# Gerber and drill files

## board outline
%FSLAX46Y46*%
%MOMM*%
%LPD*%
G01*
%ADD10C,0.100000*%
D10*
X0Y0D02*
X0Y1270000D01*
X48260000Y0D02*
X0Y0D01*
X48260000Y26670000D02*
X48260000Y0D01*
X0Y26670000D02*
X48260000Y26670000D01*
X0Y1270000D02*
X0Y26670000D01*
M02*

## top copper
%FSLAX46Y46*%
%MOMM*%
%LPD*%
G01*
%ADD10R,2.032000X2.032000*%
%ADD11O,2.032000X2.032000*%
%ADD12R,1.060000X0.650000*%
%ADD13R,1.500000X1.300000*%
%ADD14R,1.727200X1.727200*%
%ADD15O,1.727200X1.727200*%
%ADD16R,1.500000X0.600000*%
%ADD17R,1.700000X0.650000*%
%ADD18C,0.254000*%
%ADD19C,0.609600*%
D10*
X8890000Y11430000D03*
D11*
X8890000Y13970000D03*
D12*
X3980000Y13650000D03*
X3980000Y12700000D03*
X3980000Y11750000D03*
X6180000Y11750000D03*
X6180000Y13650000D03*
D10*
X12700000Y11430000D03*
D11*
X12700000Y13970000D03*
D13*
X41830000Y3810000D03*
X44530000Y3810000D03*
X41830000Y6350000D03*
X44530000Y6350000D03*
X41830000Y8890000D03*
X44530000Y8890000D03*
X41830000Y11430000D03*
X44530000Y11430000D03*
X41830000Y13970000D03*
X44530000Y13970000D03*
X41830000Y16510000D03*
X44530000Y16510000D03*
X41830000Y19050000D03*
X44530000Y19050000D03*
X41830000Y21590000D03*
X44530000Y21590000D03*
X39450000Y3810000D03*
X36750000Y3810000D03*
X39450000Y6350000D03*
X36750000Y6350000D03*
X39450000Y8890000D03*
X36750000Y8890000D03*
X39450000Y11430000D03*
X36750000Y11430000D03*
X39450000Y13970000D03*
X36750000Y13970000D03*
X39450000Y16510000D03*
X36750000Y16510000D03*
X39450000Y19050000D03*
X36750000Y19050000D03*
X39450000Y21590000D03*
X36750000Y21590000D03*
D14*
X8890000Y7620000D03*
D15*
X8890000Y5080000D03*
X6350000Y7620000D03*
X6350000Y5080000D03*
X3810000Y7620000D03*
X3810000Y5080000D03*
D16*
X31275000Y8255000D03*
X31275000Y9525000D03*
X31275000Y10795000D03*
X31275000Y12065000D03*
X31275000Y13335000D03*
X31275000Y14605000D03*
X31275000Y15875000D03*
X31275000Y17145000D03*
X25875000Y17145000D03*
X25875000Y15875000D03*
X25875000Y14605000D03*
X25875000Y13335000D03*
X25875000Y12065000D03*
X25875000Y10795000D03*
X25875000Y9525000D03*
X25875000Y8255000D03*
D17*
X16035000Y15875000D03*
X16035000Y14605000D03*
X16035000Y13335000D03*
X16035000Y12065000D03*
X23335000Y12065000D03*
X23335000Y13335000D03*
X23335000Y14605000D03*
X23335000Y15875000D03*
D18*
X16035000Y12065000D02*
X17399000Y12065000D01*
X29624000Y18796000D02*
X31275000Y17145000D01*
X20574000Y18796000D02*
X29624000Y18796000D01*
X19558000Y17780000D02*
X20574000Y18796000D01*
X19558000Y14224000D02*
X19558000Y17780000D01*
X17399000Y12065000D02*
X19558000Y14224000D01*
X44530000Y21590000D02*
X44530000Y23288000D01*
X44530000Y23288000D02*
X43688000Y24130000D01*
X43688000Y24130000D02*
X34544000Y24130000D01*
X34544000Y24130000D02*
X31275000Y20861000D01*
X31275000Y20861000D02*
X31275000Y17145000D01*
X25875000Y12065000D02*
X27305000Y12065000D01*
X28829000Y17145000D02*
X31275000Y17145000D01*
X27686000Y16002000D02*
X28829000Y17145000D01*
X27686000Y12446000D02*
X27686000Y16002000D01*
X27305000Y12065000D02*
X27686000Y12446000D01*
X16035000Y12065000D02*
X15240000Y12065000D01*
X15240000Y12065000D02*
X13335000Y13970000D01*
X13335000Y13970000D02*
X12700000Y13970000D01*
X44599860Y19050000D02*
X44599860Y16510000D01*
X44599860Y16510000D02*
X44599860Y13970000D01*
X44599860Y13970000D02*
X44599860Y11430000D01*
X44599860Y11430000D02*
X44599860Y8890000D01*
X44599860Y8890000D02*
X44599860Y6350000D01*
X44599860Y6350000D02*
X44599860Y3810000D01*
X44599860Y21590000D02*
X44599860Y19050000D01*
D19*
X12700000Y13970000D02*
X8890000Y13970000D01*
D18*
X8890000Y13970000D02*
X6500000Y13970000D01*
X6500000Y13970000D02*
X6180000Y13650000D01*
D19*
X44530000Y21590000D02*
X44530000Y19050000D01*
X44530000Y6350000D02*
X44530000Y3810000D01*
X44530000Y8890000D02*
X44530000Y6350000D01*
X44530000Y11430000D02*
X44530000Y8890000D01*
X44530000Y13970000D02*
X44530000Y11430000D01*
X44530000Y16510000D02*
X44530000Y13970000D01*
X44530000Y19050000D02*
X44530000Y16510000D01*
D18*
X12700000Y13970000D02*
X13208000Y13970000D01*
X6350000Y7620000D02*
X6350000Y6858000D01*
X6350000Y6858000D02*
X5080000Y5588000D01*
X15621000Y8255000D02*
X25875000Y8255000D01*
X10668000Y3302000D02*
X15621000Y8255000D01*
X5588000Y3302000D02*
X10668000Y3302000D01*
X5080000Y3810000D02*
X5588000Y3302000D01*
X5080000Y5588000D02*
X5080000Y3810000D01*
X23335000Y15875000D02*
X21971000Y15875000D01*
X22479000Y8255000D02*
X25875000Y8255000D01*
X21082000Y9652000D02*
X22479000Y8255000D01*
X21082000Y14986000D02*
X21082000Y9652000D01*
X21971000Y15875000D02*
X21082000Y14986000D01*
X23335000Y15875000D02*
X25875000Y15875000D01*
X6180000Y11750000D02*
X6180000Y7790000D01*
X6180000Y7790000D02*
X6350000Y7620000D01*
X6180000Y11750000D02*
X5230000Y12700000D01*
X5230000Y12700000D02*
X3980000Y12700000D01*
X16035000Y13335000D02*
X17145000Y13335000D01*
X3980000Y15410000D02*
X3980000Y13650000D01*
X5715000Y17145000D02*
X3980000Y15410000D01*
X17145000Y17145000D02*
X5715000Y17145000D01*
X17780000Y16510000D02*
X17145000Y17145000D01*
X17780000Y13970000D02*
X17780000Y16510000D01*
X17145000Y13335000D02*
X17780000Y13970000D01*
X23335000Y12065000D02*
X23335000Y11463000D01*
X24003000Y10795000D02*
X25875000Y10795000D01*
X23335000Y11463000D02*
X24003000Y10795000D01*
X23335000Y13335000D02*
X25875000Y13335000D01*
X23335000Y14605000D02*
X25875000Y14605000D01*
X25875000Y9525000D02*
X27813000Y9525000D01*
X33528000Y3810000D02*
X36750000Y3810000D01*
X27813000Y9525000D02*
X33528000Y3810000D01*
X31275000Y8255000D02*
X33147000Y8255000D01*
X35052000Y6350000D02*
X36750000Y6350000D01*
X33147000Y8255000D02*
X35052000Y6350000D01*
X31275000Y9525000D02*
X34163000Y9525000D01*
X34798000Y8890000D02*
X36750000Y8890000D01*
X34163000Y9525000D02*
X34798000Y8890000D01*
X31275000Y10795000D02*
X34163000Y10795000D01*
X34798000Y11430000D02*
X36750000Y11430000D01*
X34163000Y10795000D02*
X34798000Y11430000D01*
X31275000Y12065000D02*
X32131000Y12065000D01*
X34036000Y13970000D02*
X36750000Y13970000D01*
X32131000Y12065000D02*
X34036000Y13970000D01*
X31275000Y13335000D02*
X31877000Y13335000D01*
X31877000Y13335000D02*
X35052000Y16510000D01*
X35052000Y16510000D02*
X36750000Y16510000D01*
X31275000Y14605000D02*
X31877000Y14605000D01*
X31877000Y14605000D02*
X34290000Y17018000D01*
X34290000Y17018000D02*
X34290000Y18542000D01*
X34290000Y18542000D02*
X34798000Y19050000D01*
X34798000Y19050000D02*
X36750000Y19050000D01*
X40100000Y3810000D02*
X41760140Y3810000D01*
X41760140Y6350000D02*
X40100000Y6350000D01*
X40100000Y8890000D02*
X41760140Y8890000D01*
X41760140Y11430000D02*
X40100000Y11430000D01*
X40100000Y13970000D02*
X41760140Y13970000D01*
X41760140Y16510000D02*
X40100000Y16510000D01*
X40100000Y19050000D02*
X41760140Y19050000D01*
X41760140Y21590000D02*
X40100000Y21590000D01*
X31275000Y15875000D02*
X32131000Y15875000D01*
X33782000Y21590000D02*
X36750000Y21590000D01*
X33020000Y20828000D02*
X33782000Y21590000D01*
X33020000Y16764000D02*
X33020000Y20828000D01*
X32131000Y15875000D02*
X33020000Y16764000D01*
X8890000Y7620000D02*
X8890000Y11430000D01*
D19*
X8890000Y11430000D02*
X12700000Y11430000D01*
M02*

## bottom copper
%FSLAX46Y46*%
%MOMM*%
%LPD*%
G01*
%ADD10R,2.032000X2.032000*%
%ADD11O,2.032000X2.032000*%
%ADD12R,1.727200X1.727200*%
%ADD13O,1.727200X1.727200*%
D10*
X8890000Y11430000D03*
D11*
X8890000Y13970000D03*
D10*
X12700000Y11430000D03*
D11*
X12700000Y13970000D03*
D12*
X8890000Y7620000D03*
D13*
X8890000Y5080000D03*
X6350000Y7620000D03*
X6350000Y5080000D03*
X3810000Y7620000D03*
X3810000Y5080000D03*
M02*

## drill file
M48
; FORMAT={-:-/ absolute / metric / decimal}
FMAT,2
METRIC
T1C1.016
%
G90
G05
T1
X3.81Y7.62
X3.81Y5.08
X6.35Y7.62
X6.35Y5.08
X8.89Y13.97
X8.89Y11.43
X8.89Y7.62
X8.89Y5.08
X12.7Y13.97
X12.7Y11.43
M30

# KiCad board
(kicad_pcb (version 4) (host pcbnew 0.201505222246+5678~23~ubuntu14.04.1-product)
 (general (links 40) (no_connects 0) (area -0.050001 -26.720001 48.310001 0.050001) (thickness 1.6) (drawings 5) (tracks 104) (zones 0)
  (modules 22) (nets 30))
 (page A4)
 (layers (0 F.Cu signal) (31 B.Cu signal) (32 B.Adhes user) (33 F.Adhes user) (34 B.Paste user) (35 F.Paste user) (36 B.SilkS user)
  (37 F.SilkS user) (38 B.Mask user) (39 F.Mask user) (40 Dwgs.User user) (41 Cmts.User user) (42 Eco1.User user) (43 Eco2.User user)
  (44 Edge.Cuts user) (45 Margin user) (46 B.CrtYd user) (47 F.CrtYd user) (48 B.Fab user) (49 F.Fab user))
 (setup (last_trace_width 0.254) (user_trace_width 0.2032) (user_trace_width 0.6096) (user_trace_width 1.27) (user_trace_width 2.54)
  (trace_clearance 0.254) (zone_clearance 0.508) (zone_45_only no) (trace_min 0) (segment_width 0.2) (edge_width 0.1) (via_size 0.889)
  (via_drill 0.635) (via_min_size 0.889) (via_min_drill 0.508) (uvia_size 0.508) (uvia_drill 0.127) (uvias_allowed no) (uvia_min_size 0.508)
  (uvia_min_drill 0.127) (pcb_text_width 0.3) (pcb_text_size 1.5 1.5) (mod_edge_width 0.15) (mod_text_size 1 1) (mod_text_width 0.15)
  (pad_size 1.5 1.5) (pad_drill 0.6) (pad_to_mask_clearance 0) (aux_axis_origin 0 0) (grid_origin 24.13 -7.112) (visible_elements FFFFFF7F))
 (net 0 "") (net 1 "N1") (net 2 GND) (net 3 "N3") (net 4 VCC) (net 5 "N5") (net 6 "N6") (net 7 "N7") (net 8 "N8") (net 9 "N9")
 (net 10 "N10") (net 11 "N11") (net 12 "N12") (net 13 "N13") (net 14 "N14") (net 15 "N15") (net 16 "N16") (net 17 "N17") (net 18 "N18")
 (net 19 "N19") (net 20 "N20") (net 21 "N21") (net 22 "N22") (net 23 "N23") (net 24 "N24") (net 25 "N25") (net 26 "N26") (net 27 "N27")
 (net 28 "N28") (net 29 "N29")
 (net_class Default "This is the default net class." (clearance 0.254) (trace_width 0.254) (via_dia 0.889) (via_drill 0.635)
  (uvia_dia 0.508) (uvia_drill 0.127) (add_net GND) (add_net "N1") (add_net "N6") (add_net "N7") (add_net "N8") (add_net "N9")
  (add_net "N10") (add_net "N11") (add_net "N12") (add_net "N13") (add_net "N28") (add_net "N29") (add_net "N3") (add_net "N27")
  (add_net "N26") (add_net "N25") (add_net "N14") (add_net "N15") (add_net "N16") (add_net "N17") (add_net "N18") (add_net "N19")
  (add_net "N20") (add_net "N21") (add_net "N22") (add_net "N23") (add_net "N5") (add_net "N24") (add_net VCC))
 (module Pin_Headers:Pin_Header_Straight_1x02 (layer F.Cu) (at 8.89 -11.43 180)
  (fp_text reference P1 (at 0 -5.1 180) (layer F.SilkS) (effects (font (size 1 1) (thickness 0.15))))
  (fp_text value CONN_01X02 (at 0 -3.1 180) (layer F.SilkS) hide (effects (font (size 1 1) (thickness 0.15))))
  (pad 1 thru_hole rect (at 0 0 180) (size 2.032 2.032) (drill 1.016) (layers *.Cu *.Mask F.SilkS) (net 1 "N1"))
  (pad 2 thru_hole oval (at 0 2.54 180) (size 2.032 2.032) (drill 1.016) (layers *.Cu *.Mask F.SilkS) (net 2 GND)))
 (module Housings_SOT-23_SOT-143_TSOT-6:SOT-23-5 (layer F.Cu) (at 5.08 -12.7)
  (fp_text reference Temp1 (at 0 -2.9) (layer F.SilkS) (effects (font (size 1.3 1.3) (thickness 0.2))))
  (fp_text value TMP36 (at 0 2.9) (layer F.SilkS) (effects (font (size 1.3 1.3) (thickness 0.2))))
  (pad 1 smd rect (at -1.1 -0.95) (size 1.06 0.65) (layers F.Cu F.Paste F.Mask) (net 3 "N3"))
  (pad 2 smd rect (at -1.1 0) (size 1.06 0.65) (layers F.Cu F.Paste F.Mask) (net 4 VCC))
  (pad 3 smd rect (at -1.1 0.95) (size 1.06 0.65) (layers F.Cu F.Paste F.Mask) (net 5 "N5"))
  (pad 4 smd rect (at 1.1 0.95) (size 1.06 0.65) (layers F.Cu F.Paste F.Mask) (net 4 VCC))
  (pad 5 smd rect (at 1.1 -0.95) (size 1.06 0.65) (layers F.Cu F.Paste F.Mask) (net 2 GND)))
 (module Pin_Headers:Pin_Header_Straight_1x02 (layer F.Cu) (at 12.7 -11.43 180)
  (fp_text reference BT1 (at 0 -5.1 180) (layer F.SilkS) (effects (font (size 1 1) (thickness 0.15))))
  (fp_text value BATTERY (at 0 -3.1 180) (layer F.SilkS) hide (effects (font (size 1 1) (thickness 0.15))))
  (pad 1 thru_hole rect (at 0 0 180) (size 2.032 2.032) (drill 1.016) (layers *.Cu *.Mask F.SilkS) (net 1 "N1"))
  (pad 2 thru_hole oval (at 0 2.54 180) (size 2.032 2.032) (drill 1.016) (layers *.Cu *.Mask F.SilkS) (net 2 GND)))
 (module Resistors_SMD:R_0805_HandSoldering (layer F.Cu) (at 43.18 -3.81)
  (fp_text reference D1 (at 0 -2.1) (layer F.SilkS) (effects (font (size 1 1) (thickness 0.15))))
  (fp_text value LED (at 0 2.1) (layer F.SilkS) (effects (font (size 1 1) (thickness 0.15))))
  (pad 1 smd rect (at -1.35 0) (size 1.5 1.3) (layers F.Cu F.Paste F.Mask) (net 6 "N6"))
  (pad 2 smd rect (at 1.35 0) (size 1.5 1.3) (layers F.Cu F.Paste F.Mask) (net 2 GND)))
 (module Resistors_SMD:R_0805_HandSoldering (layer F.Cu) (at 43.18 -6.35)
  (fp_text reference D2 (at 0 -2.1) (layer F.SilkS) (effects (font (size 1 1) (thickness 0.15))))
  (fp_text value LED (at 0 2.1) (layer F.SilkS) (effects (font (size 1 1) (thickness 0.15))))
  (pad 1 smd rect (at -1.35 0) (size 1.5 1.3) (layers F.Cu F.Paste F.Mask) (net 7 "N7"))
  (pad 2 smd rect (at 1.35 0) (size 1.5 1.3) (layers F.Cu F.Paste F.Mask) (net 2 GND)))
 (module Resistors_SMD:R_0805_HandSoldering (layer F.Cu) (at 43.18 -8.89)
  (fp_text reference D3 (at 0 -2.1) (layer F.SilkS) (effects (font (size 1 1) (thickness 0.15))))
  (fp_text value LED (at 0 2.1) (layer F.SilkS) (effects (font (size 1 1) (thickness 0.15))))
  (pad 1 smd rect (at -1.35 0) (size 1.5 1.3) (layers F.Cu F.Paste F.Mask) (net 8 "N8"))
  (pad 2 smd rect (at 1.35 0) (size 1.5 1.3) (layers F.Cu F.Paste F.Mask) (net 2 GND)))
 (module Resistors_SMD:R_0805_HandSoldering (layer F.Cu) (at 43.18 -11.43)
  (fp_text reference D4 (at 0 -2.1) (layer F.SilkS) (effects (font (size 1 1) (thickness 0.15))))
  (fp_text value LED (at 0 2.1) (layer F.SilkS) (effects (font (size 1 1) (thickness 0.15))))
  (pad 1 smd rect (at -1.35 0) (size 1.5 1.3) (layers F.Cu F.Paste F.Mask) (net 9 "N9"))
  (pad 2 smd rect (at 1.35 0) (size 1.5 1.3) (layers F.Cu F.Paste F.Mask) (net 2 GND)))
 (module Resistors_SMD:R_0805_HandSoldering (layer F.Cu) (at 43.18 -13.97)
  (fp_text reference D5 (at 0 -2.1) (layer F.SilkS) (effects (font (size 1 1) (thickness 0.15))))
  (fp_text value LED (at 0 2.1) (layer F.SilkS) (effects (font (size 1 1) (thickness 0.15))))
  (pad 1 smd rect (at -1.35 0) (size 1.5 1.3) (layers F.Cu F.Paste F.Mask) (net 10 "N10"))
  (pad 2 smd rect (at 1.35 0) (size 1.5 1.3) (layers F.Cu F.Paste F.Mask) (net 2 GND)))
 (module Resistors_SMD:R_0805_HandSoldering (layer F.Cu) (at 43.18 -16.51)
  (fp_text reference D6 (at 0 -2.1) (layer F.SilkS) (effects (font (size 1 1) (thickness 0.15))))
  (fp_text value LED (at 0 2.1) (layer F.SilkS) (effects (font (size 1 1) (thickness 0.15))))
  (pad 1 smd rect (at -1.35 0) (size 1.5 1.3) (layers F.Cu F.Paste F.Mask) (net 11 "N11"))
  (pad 2 smd rect (at 1.35 0) (size 1.5 1.3) (layers F.Cu F.Paste F.Mask) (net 2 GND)))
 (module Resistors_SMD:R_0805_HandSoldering (layer F.Cu) (at 43.18 -19.05)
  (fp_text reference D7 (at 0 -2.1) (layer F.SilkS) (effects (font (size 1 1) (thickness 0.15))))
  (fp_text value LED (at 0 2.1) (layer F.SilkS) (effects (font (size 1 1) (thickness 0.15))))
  (pad 1 smd rect (at -1.35 0) (size 1.5 1.3) (layers F.Cu F.Paste F.Mask) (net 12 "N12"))
  (pad 2 smd rect (at 1.35 0) (size 1.5 1.3) (layers F.Cu F.Paste F.Mask) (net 2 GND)))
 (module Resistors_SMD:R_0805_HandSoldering (layer F.Cu) (at 43.18 -21.59)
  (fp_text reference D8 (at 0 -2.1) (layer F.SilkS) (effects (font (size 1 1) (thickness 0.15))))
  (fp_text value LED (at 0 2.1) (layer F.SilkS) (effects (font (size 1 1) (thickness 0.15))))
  (pad 1 smd rect (at -1.35 0) (size 1.5 1.3) (layers F.Cu F.Paste F.Mask) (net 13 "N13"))
  (pad 2 smd rect (at 1.35 0) (size 1.5 1.3) (layers F.Cu F.Paste F.Mask) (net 2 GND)))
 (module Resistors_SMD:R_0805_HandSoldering (layer F.Cu) (at 38.1 -3.81 180)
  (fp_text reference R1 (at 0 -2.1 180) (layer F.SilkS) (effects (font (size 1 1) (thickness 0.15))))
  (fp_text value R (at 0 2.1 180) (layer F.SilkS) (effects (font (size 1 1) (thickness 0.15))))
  (pad 1 smd rect (at -1.35 0 180) (size 1.5 1.3) (layers F.Cu F.Paste F.Mask) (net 6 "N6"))
  (pad 2 smd rect (at 1.35 0 180) (size 1.5 1.3) (layers F.Cu F.Paste F.Mask) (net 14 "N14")))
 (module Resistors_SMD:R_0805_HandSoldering (layer F.Cu) (at 38.1 -6.35 180)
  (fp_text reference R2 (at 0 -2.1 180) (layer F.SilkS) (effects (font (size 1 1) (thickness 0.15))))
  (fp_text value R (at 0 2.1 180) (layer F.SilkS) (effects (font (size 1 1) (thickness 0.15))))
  (pad 1 smd rect (at -1.35 0 180) (size 1.5 1.3) (layers F.Cu F.Paste F.Mask) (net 7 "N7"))
  (pad 2 smd rect (at 1.35 0 180) (size 1.5 1.3) (layers F.Cu F.Paste F.Mask) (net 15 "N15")))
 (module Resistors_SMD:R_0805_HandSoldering (layer F.Cu) (at 38.1 -8.89 180)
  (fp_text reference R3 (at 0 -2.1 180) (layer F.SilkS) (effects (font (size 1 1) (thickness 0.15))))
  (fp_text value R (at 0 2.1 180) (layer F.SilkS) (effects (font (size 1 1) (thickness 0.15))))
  (pad 1 smd rect (at -1.35 0 180) (size 1.5 1.3) (layers F.Cu F.Paste F.Mask) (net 8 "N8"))
  (pad 2 smd rect (at 1.35 0 180) (size 1.5 1.3) (layers F.Cu F.Paste F.Mask) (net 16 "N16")))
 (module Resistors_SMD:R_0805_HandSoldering (layer F.Cu) (at 38.1 -11.43 180)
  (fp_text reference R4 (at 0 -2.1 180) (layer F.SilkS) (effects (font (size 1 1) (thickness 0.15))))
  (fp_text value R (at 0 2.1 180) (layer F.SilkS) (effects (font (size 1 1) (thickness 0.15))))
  (pad 1 smd rect (at -1.35 0 180) (size 1.5 1.3) (layers F.Cu F.Paste F.Mask) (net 9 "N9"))
  (pad 2 smd rect (at 1.35 0 180) (size 1.5 1.3) (layers F.Cu F.Paste F.Mask) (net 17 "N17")))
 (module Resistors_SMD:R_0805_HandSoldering (layer F.Cu) (at 38.1 -13.97 180)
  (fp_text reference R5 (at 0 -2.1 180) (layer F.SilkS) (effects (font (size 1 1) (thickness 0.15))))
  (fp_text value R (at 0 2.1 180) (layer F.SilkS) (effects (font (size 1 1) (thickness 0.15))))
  (pad 1 smd rect (at -1.35 0 180) (size 1.5 1.3) (layers F.Cu F.Paste F.Mask) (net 10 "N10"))
  (pad 2 smd rect (at 1.35 0 180) (size 1.5 1.3) (layers F.Cu F.Paste F.Mask) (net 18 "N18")))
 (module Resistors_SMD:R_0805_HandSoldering (layer F.Cu) (at 38.1 -16.51 180)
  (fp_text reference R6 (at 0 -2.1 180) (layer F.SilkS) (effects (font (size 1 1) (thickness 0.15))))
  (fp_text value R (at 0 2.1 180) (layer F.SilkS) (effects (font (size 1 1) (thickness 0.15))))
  (pad 1 smd rect (at -1.35 0 180) (size 1.5 1.3) (layers F.Cu F.Paste F.Mask) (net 11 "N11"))
  (pad 2 smd rect (at 1.35 0 180) (size 1.5 1.3) (layers F.Cu F.Paste F.Mask) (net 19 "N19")))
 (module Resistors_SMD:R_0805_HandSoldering (layer F.Cu) (at 38.1 -19.05 180)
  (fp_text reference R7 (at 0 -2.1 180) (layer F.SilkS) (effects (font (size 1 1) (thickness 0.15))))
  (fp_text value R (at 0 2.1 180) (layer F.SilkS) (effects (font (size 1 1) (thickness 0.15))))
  (pad 1 smd rect (at -1.35 0 180) (size 1.5 1.3) (layers F.Cu F.Paste F.Mask) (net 12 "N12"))
  (pad 2 smd rect (at 1.35 0 180) (size 1.5 1.3) (layers F.Cu F.Paste F.Mask) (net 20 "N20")))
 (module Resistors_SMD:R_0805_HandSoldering (layer F.Cu) (at 38.1 -21.59 180)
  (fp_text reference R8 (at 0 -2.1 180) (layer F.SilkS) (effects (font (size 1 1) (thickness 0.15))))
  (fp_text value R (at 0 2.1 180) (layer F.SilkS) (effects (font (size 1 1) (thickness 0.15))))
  (pad 1 smd rect (at -1.35 0 180) (size 1.5 1.3) (layers F.Cu F.Paste F.Mask) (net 13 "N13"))
  (pad 2 smd rect (at 1.35 0 180) (size 1.5 1.3) (layers F.Cu F.Paste F.Mask) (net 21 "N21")))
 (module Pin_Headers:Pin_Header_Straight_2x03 (layer F.Cu) (at 8.89 -7.62 270)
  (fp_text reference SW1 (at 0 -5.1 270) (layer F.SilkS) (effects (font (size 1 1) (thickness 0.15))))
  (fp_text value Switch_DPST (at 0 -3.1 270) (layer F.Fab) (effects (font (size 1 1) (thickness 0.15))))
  (pad 1 thru_hole rect (at 0 0 270) (size 1.7272 1.7272) (drill 1.016) (layers *.Cu *.Mask F.SilkS) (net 1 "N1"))
  (pad 2 thru_hole oval (at 2.54 0 270) (size 1.7272 1.7272) (drill 1.016) (layers *.Cu *.Mask F.SilkS) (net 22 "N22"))
  (pad 3 thru_hole oval (at 0 2.54 270) (size 1.7272 1.7272) (drill 1.016) (layers *.Cu *.Mask F.SilkS) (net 4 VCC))
  (pad 4 thru_hole oval (at 2.54 2.54 270) (size 1.7272 1.7272) (drill 1.016) (layers *.Cu *.Mask F.SilkS) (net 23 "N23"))
  (pad 5 thru_hole oval (at 0 5.08 270) (size 1.7272 1.7272) (drill 1.016) (layers *.Cu *.Mask F.SilkS))
  (pad 6 thru_hole oval (at 2.54 5.08 270) (size 1.7272 1.7272) (drill 1.016) (layers *.Cu *.Mask F.SilkS)))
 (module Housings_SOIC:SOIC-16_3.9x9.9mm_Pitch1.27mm (layer F.Cu) (at 28.575 -12.7 180)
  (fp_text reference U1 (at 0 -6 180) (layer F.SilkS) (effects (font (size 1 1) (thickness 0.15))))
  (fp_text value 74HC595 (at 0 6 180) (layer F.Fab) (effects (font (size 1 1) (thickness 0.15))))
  (pad 1 smd rect (at -2.7 -4.445 180) (size 1.5 0.6) (layers F.Cu F.Paste F.Mask) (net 15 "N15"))
  (pad 2 smd rect (at -2.7 -3.175 180) (size 1.5 0.6) (layers F.Cu F.Paste F.Mask) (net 16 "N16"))
  (pad 3 smd rect (at -2.7 -1.905 180) (size 1.5 0.6) (layers F.Cu F.Paste F.Mask) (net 17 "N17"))
  (pad 4 smd rect (at -2.7 -0.635 180) (size 1.5 0.6) (layers F.Cu F.Paste F.Mask) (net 18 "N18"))
  (pad 5 smd rect (at -2.7 0.635 180) (size 1.5 0.6) (layers F.Cu F.Paste F.Mask) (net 19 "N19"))
  (pad 6 smd rect (at -2.7 1.905 180) (size 1.5 0.6) (layers F.Cu F.Paste F.Mask) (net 20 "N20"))
  (pad 7 smd rect (at -2.7 3.175 180) (size 1.5 0.6) (layers F.Cu F.Paste F.Mask) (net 21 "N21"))
  (pad 8 smd rect (at -2.7 4.445 180) (size 1.5 0.6) (layers F.Cu F.Paste F.Mask) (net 2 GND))
  (pad 9 smd rect (at 2.7 4.445 180) (size 1.5 0.6) (layers F.Cu F.Paste F.Mask) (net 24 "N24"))
  (pad 10 smd rect (at 2.7 3.175 180) (size 1.5 0.6) (layers F.Cu F.Paste F.Mask) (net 4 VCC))
  (pad 11 smd rect (at 2.7 1.905 180) (size 1.5 0.6) (layers F.Cu F.Paste F.Mask) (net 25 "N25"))
  (pad 12 smd rect (at 2.7 0.635 180) (size 1.5 0.6) (layers F.Cu F.Paste F.Mask) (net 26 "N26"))
  (pad 13 smd rect (at 2.7 -0.635 180) (size 1.5 0.6) (layers F.Cu F.Paste F.Mask) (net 2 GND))
  (pad 14 smd rect (at 2.7 -1.905 180) (size 1.5 0.6) (layers F.Cu F.Paste F.Mask) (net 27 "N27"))
  (pad 15 smd rect (at 2.7 -3.175 180) (size 1.5 0.6) (layers F.Cu F.Paste F.Mask) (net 14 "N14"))
  (pad 16 smd rect (at 2.7 -4.445 180) (size 1.5 0.6) (layers F.Cu F.Paste F.Mask) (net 4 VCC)))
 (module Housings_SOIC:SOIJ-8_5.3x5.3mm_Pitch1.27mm (layer F.Cu) (at 19.685 -13.97)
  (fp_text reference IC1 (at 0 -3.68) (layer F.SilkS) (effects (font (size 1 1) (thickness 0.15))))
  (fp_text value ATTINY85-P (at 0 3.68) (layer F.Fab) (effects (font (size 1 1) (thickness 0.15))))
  (pad 1 smd rect (at -3.65 -1.905) (size 1.7 0.65) (layers F.Cu F.Paste F.Mask) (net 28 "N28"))
  (pad 2 smd rect (at -3.65 -0.635) (size 1.7 0.65) (layers F.Cu F.Paste F.Mask) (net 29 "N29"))
  (pad 3 smd rect (at -3.65 0.635) (size 1.7 0.65) (layers F.Cu F.Paste F.Mask) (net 3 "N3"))
  (pad 4 smd rect (at -3.65 1.905) (size 1.7 0.65) (layers F.Cu F.Paste F.Mask) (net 2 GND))
  (pad 5 smd rect (at 3.65 1.905) (size 1.7 0.65) (layers F.Cu F.Paste F.Mask) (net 27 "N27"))
  (pad 6 smd rect (at 3.65 0.635) (size 1.7 0.65) (layers F.Cu F.Paste F.Mask) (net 26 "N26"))
  (pad 7 smd rect (at 3.65 -0.635) (size 1.7 0.65) (layers F.Cu F.Paste F.Mask) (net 25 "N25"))
  (pad 8 smd rect (at 3.65 -1.905) (size 1.7 0.65) (layers F.Cu F.Paste F.Mask) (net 4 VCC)))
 (gr_line (start 0 0) (end 0 -1.27) (angle 90) (layer Edge.Cuts) (width 0.1))
 (gr_line (start 48.26 0) (end 0 0) (angle 90) (layer Edge.Cuts) (width 0.1))
 (gr_line (start 48.26 -26.67) (end 48.26 0) (angle 90) (layer Edge.Cuts) (width 0.1))
 (gr_line (start 0 -26.67) (end 48.26 -26.67) (angle 90) (layer Edge.Cuts) (width 0.1))
 (gr_line (start 0 -1.27) (end 0 -26.67) (angle 90) (layer Edge.Cuts) (width 0.1))
 (segment (start 16.035 -12.065) (end 17.399 -12.065) (width 0.254) (layer F.Cu) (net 2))
 (segment (start 29.624 -18.796) (end 31.275 -17.145) (width 0.254) (layer F.Cu) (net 2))
 (segment (start 20.574 -18.796) (end 29.624 -18.796) (width 0.254) (layer F.Cu) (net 2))
 (segment (start 19.558 -17.78) (end 20.574 -18.796) (width 0.254) (layer F.Cu) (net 2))
 (segment (start 19.558 -14.224) (end 19.558 -17.78) (width 0.254) (layer F.Cu) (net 2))
 (segment (start 17.399 -12.065) (end 19.558 -14.224) (width 0.254) (layer F.Cu) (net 2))
 (segment (start 44.53 -21.59) (end 44.53 -23.288) (width 0.254) (layer F.Cu) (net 2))
 (segment (start 44.53 -23.288) (end 43.688 -24.13) (width 0.254) (layer F.Cu) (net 2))
 (segment (start 43.688 -24.13) (end 34.544 -24.13) (width 0.254) (layer F.Cu) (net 2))
 (segment (start 34.544 -24.13) (end 31.275 -20.861) (width 0.254) (layer F.Cu) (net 2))
 (segment (start 31.275 -20.861) (end 31.275 -17.145) (width 0.254) (layer F.Cu) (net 2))
 (segment (start 25.875 -12.065) (end 27.305 -12.065) (width 0.254) (layer F.Cu) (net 2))
 (segment (start 28.829 -17.145) (end 31.275 -17.145) (width 0.254) (layer F.Cu) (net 2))
 (segment (start 27.686 -16.002) (end 28.829 -17.145) (width 0.254) (layer F.Cu) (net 2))
 (segment (start 27.686 -12.446) (end 27.686 -16.002) (width 0.254) (layer F.Cu) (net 2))
 (segment (start 27.305 -12.065) (end 27.686 -12.446) (width 0.254) (layer F.Cu) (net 2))
 (segment (start 16.035 -12.065) (end 15.24 -12.065) (width 0.254) (layer F.Cu) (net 2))
 (segment (start 15.24 -12.065) (end 13.335 -13.97) (width 0.254) (layer F.Cu) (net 2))
 (segment (start 13.335 -13.97) (end 12.7 -13.97) (width 0.254) (layer F.Cu) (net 2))
 (segment (start 44.59986 -19.05) (end 44.59986 -16.51) (width 0.254) (layer F.Cu) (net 2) (status 20))
 (segment (start 44.59986 -16.51) (end 44.59986 -13.97) (width 0.254) (layer F.Cu) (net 2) (status 20))
 (segment (start 44.59986 -13.97) (end 44.59986 -11.43) (width 0.254) (layer F.Cu) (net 2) (status 20))
 (segment (start 44.59986 -11.43) (end 44.59986 -8.89) (width 0.254) (layer F.Cu) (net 2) (status 20))
 (segment (start 44.59986 -8.89) (end 44.59986 -6.35) (width 0.254) (layer F.Cu) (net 2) (status 20))
 (segment (start 44.59986 -6.35) (end 44.59986 -3.81) (width 0.254) (layer F.Cu) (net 2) (status 20))
 (segment (start 44.59986 -21.59) (end 44.59986 -19.05) (width 0.254) (layer F.Cu) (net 2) (status 20))
 (segment (start 12.7 -13.97) (end 8.89 -13.97) (width 0.6096) (layer F.Cu) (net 2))
 (segment (start 8.89 -13.97) (end 6.5 -13.97) (width 0.254) (layer F.Cu) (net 2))
 (segment (start 6.5 -13.97) (end 6.18 -13.65) (width 0.254) (layer F.Cu) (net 2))
 (segment (start 44.53 -21.59) (end 44.53 -19.05) (width 0.6096) (layer F.Cu) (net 2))
 (segment (start 44.53 -6.35) (end 44.53 -3.81) (width 0.6096) (layer F.Cu) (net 2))
 (segment (start 44.53 -8.89) (end 44.53 -6.35) (width 0.6096) (layer F.Cu) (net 2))
 (segment (start 44.53 -11.43) (end 44.53 -8.89) (width 0.6096) (layer F.Cu) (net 2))
 (segment (start 44.53 -13.97) (end 44.53 -11.43) (width 0.6096) (layer F.Cu) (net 2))
 (segment (start 44.53 -16.51) (end 44.53 -13.97) (width 0.6096) (layer F.Cu) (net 2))
 (segment (start 44.53 -19.05) (end 44.53 -16.51) (width 0.6096) (layer F.Cu) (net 2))
 (segment (start 12.7 -13.97) (end 13.208 -13.97) (width 0.254) (layer F.Cu) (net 2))
 (segment (start 6.35 -7.62) (end 6.35 -6.858) (width 0.254) (layer F.Cu) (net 4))
 (segment (start 6.35 -6.858) (end 5.08 -5.588) (width 0.254) (layer F.Cu) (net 4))
 (segment (start 15.621 -8.255) (end 25.875 -8.255) (width 0.254) (layer F.Cu) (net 4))
 (segment (start 10.668 -3.302) (end 15.621 -8.255) (width 0.254) (layer F.Cu) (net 4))
 (segment (start 5.588 -3.302) (end 10.668 -3.302) (width 0.254) (layer F.Cu) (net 4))
 (segment (start 5.08 -3.81) (end 5.588 -3.302) (width 0.254) (layer F.Cu) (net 4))
 (segment (start 5.08 -5.588) (end 5.08 -3.81) (width 0.254) (layer F.Cu) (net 4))
 (segment (start 23.335 -15.875) (end 21.971 -15.875) (width 0.254) (layer F.Cu) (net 4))
 (segment (start 22.479 -8.255) (end 25.875 -8.255) (width 0.254) (layer F.Cu) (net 4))
 (segment (start 21.082 -9.652) (end 22.479 -8.255) (width 0.254) (layer F.Cu) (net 4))
 (segment (start 21.082 -14.986) (end 21.082 -9.652) (width 0.254) (layer F.Cu) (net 4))
 (segment (start 21.971 -15.875) (end 21.082 -14.986) (width 0.254) (layer F.Cu) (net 4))
 (segment (start 23.335 -15.875) (end 25.875 -15.875) (width 0.254) (layer F.Cu) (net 4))
 (segment (start 6.18 -11.75) (end 6.18 -7.79) (width 0.254) (layer F.Cu) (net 4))
 (segment (start 6.18 -7.79) (end 6.35 -7.62) (width 0.254) (layer F.Cu) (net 4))
 (segment (start 6.18 -11.75) (end 5.23 -12.7) (width 0.254) (layer F.Cu) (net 4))
 (segment (start 5.23 -12.7) (end 3.98 -12.7) (width 0.254) (layer F.Cu) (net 4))
 (segment (start 16.035 -13.335) (end 17.145 -13.335) (width 0.254) (layer F.Cu) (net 3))
 (segment (start 3.98 -15.41) (end 3.98 -13.65) (width 0.254) (layer F.Cu) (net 3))
 (segment (start 5.715 -17.145) (end 3.98 -15.41) (width 0.254) (layer F.Cu) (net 3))
 (segment (start 17.145 -17.145) (end 5.715 -17.145) (width 0.254) (layer F.Cu) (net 3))
 (segment (start 17.78 -16.51) (end 17.145 -17.145) (width 0.254) (layer F.Cu) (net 3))
 (segment (start 17.78 -13.97) (end 17.78 -16.51) (width 0.254) (layer F.Cu) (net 3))
 (segment (start 17.145 -13.335) (end 17.78 -13.97) (width 0.254) (layer F.Cu) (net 3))
 (segment (start 23.335 -12.065) (end 23.335 -11.463) (width 0.254) (layer F.Cu) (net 27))
 (segment (start 24.003 -10.795) (end 25.875 -10.795) (width 0.254) (layer F.Cu) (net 27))
 (segment (start 23.335 -11.463) (end 24.003 -10.795) (width 0.254) (layer F.Cu) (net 27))
 (segment (start 23.335 -13.335) (end 25.875 -13.335) (width 0.254) (layer F.Cu) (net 26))
 (segment (start 23.335 -14.605) (end 25.875 -14.605) (width 0.254) (layer F.Cu) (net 25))
 (segment (start 25.875 -9.525) (end 27.813 -9.525) (width 0.254) (layer F.Cu) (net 14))
 (segment (start 33.528 -3.81) (end 36.75 -3.81) (width 0.254) (layer F.Cu) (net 14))
 (segment (start 27.813 -9.525) (end 33.528 -3.81) (width 0.254) (layer F.Cu) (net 14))
 (segment (start 31.275 -8.255) (end 33.147 -8.255) (width 0.254) (layer F.Cu) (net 15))
 (segment (start 35.052 -6.35) (end 36.75 -6.35) (width 0.254) (layer F.Cu) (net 15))
 (segment (start 33.147 -8.255) (end 35.052 -6.35) (width 0.254) (layer F.Cu) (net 15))
 (segment (start 31.275 -9.525) (end 34.163 -9.525) (width 0.254) (layer F.Cu) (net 16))
 (segment (start 34.798 -8.89) (end 36.75 -8.89) (width 0.254) (layer F.Cu) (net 16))
 (segment (start 34.163 -9.525) (end 34.798 -8.89) (width 0.254) (layer F.Cu) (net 16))
 (segment (start 31.275 -10.795) (end 34.163 -10.795) (width 0.254) (layer F.Cu) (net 17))
 (segment (start 34.798 -11.43) (end 36.75 -11.43) (width 0.254) (layer F.Cu) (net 17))
 (segment (start 34.163 -10.795) (end 34.798 -11.43) (width 0.254) (layer F.Cu) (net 17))
 (segment (start 31.275 -12.065) (end 32.131 -12.065) (width 0.254) (layer F.Cu) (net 18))
 (segment (start 34.036 -13.97) (end 36.75 -13.97) (width 0.254) (layer F.Cu) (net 18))
 (segment (start 32.131 -12.065) (end 34.036 -13.97) (width 0.254) (layer F.Cu) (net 18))
 (segment (start 31.275 -13.335) (end 31.877 -13.335) (width 0.254) (layer F.Cu) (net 19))
 (segment (start 31.877 -13.335) (end 35.052 -16.51) (width 0.254) (layer F.Cu) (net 19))
 (segment (start 35.052 -16.51) (end 36.75 -16.51) (width 0.254) (layer F.Cu) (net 19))
 (segment (start 31.275 -14.605) (end 31.877 -14.605) (width 0.254) (layer F.Cu) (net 20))
 (segment (start 31.877 -14.605) (end 34.29 -17.018) (width 0.254) (layer F.Cu) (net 20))
 (segment (start 34.29 -17.018) (end 34.29 -18.542) (width 0.254) (layer F.Cu) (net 20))
 (segment (start 34.29 -18.542) (end 34.798 -19.05) (width 0.254) (layer F.Cu) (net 20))
 (segment (start 34.798 -19.05) (end 36.75 -19.05) (width 0.254) (layer F.Cu) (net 20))
 (segment (start 40.1 -3.81) (end 41.76014 -3.81) (width 0.254) (layer F.Cu) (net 6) (status 20))
 (segment (start 41.76014 -6.35) (end 40.1 -6.35) (width 0.254) (layer F.Cu) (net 7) (status 10))
 (segment (start 40.1 -8.89) (end 41.76014 -8.89) (width 0.254) (layer F.Cu) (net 8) (status 20))
 (segment (start 41.76014 -11.43) (end 40.1 -11.43) (width 0.254) (layer F.Cu) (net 9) (status 20))
 (segment (start 40.1 -13.97) (end 41.76014 -13.97) (width 0.254) (layer F.Cu) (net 10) (status 20))
 (segment (start 41.76014 -16.51) (end 40.1 -16.51) (width 0.254) (layer F.Cu) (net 11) (status 20))
 (segment (start 40.1 -19.05) (end 41.76014 -19.05) (width 0.254) (layer F.Cu) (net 12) (status 20))
 (segment (start 41.76014 -21.59) (end 40.1 -21.59) (width 0.254) (layer F.Cu) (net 13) (status 10))
 (segment (start 31.275 -15.875) (end 32.131 -15.875) (width 0.254) (layer F.Cu) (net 21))
 (segment (start 33.782 -21.59) (end 36.75 -21.59) (width 0.254) (layer F.Cu) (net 21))
 (segment (start 33.02 -20.828) (end 33.782 -21.59) (width 0.254) (layer F.Cu) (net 21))
 (segment (start 33.02 -16.764) (end 33.02 -20.828) (width 0.254) (layer F.Cu) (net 21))
 (segment (start 32.131 -15.875) (end 33.02 -16.764) (width 0.254) (layer F.Cu) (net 21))
 (segment (start 8.89 -7.62) (end 8.89 -11.43) (width 0.254) (layer F.Cu) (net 1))
 (segment (start 8.89 -11.43) (end 12.7 -11.43) (width 0.6096) (layer F.Cu) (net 1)))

